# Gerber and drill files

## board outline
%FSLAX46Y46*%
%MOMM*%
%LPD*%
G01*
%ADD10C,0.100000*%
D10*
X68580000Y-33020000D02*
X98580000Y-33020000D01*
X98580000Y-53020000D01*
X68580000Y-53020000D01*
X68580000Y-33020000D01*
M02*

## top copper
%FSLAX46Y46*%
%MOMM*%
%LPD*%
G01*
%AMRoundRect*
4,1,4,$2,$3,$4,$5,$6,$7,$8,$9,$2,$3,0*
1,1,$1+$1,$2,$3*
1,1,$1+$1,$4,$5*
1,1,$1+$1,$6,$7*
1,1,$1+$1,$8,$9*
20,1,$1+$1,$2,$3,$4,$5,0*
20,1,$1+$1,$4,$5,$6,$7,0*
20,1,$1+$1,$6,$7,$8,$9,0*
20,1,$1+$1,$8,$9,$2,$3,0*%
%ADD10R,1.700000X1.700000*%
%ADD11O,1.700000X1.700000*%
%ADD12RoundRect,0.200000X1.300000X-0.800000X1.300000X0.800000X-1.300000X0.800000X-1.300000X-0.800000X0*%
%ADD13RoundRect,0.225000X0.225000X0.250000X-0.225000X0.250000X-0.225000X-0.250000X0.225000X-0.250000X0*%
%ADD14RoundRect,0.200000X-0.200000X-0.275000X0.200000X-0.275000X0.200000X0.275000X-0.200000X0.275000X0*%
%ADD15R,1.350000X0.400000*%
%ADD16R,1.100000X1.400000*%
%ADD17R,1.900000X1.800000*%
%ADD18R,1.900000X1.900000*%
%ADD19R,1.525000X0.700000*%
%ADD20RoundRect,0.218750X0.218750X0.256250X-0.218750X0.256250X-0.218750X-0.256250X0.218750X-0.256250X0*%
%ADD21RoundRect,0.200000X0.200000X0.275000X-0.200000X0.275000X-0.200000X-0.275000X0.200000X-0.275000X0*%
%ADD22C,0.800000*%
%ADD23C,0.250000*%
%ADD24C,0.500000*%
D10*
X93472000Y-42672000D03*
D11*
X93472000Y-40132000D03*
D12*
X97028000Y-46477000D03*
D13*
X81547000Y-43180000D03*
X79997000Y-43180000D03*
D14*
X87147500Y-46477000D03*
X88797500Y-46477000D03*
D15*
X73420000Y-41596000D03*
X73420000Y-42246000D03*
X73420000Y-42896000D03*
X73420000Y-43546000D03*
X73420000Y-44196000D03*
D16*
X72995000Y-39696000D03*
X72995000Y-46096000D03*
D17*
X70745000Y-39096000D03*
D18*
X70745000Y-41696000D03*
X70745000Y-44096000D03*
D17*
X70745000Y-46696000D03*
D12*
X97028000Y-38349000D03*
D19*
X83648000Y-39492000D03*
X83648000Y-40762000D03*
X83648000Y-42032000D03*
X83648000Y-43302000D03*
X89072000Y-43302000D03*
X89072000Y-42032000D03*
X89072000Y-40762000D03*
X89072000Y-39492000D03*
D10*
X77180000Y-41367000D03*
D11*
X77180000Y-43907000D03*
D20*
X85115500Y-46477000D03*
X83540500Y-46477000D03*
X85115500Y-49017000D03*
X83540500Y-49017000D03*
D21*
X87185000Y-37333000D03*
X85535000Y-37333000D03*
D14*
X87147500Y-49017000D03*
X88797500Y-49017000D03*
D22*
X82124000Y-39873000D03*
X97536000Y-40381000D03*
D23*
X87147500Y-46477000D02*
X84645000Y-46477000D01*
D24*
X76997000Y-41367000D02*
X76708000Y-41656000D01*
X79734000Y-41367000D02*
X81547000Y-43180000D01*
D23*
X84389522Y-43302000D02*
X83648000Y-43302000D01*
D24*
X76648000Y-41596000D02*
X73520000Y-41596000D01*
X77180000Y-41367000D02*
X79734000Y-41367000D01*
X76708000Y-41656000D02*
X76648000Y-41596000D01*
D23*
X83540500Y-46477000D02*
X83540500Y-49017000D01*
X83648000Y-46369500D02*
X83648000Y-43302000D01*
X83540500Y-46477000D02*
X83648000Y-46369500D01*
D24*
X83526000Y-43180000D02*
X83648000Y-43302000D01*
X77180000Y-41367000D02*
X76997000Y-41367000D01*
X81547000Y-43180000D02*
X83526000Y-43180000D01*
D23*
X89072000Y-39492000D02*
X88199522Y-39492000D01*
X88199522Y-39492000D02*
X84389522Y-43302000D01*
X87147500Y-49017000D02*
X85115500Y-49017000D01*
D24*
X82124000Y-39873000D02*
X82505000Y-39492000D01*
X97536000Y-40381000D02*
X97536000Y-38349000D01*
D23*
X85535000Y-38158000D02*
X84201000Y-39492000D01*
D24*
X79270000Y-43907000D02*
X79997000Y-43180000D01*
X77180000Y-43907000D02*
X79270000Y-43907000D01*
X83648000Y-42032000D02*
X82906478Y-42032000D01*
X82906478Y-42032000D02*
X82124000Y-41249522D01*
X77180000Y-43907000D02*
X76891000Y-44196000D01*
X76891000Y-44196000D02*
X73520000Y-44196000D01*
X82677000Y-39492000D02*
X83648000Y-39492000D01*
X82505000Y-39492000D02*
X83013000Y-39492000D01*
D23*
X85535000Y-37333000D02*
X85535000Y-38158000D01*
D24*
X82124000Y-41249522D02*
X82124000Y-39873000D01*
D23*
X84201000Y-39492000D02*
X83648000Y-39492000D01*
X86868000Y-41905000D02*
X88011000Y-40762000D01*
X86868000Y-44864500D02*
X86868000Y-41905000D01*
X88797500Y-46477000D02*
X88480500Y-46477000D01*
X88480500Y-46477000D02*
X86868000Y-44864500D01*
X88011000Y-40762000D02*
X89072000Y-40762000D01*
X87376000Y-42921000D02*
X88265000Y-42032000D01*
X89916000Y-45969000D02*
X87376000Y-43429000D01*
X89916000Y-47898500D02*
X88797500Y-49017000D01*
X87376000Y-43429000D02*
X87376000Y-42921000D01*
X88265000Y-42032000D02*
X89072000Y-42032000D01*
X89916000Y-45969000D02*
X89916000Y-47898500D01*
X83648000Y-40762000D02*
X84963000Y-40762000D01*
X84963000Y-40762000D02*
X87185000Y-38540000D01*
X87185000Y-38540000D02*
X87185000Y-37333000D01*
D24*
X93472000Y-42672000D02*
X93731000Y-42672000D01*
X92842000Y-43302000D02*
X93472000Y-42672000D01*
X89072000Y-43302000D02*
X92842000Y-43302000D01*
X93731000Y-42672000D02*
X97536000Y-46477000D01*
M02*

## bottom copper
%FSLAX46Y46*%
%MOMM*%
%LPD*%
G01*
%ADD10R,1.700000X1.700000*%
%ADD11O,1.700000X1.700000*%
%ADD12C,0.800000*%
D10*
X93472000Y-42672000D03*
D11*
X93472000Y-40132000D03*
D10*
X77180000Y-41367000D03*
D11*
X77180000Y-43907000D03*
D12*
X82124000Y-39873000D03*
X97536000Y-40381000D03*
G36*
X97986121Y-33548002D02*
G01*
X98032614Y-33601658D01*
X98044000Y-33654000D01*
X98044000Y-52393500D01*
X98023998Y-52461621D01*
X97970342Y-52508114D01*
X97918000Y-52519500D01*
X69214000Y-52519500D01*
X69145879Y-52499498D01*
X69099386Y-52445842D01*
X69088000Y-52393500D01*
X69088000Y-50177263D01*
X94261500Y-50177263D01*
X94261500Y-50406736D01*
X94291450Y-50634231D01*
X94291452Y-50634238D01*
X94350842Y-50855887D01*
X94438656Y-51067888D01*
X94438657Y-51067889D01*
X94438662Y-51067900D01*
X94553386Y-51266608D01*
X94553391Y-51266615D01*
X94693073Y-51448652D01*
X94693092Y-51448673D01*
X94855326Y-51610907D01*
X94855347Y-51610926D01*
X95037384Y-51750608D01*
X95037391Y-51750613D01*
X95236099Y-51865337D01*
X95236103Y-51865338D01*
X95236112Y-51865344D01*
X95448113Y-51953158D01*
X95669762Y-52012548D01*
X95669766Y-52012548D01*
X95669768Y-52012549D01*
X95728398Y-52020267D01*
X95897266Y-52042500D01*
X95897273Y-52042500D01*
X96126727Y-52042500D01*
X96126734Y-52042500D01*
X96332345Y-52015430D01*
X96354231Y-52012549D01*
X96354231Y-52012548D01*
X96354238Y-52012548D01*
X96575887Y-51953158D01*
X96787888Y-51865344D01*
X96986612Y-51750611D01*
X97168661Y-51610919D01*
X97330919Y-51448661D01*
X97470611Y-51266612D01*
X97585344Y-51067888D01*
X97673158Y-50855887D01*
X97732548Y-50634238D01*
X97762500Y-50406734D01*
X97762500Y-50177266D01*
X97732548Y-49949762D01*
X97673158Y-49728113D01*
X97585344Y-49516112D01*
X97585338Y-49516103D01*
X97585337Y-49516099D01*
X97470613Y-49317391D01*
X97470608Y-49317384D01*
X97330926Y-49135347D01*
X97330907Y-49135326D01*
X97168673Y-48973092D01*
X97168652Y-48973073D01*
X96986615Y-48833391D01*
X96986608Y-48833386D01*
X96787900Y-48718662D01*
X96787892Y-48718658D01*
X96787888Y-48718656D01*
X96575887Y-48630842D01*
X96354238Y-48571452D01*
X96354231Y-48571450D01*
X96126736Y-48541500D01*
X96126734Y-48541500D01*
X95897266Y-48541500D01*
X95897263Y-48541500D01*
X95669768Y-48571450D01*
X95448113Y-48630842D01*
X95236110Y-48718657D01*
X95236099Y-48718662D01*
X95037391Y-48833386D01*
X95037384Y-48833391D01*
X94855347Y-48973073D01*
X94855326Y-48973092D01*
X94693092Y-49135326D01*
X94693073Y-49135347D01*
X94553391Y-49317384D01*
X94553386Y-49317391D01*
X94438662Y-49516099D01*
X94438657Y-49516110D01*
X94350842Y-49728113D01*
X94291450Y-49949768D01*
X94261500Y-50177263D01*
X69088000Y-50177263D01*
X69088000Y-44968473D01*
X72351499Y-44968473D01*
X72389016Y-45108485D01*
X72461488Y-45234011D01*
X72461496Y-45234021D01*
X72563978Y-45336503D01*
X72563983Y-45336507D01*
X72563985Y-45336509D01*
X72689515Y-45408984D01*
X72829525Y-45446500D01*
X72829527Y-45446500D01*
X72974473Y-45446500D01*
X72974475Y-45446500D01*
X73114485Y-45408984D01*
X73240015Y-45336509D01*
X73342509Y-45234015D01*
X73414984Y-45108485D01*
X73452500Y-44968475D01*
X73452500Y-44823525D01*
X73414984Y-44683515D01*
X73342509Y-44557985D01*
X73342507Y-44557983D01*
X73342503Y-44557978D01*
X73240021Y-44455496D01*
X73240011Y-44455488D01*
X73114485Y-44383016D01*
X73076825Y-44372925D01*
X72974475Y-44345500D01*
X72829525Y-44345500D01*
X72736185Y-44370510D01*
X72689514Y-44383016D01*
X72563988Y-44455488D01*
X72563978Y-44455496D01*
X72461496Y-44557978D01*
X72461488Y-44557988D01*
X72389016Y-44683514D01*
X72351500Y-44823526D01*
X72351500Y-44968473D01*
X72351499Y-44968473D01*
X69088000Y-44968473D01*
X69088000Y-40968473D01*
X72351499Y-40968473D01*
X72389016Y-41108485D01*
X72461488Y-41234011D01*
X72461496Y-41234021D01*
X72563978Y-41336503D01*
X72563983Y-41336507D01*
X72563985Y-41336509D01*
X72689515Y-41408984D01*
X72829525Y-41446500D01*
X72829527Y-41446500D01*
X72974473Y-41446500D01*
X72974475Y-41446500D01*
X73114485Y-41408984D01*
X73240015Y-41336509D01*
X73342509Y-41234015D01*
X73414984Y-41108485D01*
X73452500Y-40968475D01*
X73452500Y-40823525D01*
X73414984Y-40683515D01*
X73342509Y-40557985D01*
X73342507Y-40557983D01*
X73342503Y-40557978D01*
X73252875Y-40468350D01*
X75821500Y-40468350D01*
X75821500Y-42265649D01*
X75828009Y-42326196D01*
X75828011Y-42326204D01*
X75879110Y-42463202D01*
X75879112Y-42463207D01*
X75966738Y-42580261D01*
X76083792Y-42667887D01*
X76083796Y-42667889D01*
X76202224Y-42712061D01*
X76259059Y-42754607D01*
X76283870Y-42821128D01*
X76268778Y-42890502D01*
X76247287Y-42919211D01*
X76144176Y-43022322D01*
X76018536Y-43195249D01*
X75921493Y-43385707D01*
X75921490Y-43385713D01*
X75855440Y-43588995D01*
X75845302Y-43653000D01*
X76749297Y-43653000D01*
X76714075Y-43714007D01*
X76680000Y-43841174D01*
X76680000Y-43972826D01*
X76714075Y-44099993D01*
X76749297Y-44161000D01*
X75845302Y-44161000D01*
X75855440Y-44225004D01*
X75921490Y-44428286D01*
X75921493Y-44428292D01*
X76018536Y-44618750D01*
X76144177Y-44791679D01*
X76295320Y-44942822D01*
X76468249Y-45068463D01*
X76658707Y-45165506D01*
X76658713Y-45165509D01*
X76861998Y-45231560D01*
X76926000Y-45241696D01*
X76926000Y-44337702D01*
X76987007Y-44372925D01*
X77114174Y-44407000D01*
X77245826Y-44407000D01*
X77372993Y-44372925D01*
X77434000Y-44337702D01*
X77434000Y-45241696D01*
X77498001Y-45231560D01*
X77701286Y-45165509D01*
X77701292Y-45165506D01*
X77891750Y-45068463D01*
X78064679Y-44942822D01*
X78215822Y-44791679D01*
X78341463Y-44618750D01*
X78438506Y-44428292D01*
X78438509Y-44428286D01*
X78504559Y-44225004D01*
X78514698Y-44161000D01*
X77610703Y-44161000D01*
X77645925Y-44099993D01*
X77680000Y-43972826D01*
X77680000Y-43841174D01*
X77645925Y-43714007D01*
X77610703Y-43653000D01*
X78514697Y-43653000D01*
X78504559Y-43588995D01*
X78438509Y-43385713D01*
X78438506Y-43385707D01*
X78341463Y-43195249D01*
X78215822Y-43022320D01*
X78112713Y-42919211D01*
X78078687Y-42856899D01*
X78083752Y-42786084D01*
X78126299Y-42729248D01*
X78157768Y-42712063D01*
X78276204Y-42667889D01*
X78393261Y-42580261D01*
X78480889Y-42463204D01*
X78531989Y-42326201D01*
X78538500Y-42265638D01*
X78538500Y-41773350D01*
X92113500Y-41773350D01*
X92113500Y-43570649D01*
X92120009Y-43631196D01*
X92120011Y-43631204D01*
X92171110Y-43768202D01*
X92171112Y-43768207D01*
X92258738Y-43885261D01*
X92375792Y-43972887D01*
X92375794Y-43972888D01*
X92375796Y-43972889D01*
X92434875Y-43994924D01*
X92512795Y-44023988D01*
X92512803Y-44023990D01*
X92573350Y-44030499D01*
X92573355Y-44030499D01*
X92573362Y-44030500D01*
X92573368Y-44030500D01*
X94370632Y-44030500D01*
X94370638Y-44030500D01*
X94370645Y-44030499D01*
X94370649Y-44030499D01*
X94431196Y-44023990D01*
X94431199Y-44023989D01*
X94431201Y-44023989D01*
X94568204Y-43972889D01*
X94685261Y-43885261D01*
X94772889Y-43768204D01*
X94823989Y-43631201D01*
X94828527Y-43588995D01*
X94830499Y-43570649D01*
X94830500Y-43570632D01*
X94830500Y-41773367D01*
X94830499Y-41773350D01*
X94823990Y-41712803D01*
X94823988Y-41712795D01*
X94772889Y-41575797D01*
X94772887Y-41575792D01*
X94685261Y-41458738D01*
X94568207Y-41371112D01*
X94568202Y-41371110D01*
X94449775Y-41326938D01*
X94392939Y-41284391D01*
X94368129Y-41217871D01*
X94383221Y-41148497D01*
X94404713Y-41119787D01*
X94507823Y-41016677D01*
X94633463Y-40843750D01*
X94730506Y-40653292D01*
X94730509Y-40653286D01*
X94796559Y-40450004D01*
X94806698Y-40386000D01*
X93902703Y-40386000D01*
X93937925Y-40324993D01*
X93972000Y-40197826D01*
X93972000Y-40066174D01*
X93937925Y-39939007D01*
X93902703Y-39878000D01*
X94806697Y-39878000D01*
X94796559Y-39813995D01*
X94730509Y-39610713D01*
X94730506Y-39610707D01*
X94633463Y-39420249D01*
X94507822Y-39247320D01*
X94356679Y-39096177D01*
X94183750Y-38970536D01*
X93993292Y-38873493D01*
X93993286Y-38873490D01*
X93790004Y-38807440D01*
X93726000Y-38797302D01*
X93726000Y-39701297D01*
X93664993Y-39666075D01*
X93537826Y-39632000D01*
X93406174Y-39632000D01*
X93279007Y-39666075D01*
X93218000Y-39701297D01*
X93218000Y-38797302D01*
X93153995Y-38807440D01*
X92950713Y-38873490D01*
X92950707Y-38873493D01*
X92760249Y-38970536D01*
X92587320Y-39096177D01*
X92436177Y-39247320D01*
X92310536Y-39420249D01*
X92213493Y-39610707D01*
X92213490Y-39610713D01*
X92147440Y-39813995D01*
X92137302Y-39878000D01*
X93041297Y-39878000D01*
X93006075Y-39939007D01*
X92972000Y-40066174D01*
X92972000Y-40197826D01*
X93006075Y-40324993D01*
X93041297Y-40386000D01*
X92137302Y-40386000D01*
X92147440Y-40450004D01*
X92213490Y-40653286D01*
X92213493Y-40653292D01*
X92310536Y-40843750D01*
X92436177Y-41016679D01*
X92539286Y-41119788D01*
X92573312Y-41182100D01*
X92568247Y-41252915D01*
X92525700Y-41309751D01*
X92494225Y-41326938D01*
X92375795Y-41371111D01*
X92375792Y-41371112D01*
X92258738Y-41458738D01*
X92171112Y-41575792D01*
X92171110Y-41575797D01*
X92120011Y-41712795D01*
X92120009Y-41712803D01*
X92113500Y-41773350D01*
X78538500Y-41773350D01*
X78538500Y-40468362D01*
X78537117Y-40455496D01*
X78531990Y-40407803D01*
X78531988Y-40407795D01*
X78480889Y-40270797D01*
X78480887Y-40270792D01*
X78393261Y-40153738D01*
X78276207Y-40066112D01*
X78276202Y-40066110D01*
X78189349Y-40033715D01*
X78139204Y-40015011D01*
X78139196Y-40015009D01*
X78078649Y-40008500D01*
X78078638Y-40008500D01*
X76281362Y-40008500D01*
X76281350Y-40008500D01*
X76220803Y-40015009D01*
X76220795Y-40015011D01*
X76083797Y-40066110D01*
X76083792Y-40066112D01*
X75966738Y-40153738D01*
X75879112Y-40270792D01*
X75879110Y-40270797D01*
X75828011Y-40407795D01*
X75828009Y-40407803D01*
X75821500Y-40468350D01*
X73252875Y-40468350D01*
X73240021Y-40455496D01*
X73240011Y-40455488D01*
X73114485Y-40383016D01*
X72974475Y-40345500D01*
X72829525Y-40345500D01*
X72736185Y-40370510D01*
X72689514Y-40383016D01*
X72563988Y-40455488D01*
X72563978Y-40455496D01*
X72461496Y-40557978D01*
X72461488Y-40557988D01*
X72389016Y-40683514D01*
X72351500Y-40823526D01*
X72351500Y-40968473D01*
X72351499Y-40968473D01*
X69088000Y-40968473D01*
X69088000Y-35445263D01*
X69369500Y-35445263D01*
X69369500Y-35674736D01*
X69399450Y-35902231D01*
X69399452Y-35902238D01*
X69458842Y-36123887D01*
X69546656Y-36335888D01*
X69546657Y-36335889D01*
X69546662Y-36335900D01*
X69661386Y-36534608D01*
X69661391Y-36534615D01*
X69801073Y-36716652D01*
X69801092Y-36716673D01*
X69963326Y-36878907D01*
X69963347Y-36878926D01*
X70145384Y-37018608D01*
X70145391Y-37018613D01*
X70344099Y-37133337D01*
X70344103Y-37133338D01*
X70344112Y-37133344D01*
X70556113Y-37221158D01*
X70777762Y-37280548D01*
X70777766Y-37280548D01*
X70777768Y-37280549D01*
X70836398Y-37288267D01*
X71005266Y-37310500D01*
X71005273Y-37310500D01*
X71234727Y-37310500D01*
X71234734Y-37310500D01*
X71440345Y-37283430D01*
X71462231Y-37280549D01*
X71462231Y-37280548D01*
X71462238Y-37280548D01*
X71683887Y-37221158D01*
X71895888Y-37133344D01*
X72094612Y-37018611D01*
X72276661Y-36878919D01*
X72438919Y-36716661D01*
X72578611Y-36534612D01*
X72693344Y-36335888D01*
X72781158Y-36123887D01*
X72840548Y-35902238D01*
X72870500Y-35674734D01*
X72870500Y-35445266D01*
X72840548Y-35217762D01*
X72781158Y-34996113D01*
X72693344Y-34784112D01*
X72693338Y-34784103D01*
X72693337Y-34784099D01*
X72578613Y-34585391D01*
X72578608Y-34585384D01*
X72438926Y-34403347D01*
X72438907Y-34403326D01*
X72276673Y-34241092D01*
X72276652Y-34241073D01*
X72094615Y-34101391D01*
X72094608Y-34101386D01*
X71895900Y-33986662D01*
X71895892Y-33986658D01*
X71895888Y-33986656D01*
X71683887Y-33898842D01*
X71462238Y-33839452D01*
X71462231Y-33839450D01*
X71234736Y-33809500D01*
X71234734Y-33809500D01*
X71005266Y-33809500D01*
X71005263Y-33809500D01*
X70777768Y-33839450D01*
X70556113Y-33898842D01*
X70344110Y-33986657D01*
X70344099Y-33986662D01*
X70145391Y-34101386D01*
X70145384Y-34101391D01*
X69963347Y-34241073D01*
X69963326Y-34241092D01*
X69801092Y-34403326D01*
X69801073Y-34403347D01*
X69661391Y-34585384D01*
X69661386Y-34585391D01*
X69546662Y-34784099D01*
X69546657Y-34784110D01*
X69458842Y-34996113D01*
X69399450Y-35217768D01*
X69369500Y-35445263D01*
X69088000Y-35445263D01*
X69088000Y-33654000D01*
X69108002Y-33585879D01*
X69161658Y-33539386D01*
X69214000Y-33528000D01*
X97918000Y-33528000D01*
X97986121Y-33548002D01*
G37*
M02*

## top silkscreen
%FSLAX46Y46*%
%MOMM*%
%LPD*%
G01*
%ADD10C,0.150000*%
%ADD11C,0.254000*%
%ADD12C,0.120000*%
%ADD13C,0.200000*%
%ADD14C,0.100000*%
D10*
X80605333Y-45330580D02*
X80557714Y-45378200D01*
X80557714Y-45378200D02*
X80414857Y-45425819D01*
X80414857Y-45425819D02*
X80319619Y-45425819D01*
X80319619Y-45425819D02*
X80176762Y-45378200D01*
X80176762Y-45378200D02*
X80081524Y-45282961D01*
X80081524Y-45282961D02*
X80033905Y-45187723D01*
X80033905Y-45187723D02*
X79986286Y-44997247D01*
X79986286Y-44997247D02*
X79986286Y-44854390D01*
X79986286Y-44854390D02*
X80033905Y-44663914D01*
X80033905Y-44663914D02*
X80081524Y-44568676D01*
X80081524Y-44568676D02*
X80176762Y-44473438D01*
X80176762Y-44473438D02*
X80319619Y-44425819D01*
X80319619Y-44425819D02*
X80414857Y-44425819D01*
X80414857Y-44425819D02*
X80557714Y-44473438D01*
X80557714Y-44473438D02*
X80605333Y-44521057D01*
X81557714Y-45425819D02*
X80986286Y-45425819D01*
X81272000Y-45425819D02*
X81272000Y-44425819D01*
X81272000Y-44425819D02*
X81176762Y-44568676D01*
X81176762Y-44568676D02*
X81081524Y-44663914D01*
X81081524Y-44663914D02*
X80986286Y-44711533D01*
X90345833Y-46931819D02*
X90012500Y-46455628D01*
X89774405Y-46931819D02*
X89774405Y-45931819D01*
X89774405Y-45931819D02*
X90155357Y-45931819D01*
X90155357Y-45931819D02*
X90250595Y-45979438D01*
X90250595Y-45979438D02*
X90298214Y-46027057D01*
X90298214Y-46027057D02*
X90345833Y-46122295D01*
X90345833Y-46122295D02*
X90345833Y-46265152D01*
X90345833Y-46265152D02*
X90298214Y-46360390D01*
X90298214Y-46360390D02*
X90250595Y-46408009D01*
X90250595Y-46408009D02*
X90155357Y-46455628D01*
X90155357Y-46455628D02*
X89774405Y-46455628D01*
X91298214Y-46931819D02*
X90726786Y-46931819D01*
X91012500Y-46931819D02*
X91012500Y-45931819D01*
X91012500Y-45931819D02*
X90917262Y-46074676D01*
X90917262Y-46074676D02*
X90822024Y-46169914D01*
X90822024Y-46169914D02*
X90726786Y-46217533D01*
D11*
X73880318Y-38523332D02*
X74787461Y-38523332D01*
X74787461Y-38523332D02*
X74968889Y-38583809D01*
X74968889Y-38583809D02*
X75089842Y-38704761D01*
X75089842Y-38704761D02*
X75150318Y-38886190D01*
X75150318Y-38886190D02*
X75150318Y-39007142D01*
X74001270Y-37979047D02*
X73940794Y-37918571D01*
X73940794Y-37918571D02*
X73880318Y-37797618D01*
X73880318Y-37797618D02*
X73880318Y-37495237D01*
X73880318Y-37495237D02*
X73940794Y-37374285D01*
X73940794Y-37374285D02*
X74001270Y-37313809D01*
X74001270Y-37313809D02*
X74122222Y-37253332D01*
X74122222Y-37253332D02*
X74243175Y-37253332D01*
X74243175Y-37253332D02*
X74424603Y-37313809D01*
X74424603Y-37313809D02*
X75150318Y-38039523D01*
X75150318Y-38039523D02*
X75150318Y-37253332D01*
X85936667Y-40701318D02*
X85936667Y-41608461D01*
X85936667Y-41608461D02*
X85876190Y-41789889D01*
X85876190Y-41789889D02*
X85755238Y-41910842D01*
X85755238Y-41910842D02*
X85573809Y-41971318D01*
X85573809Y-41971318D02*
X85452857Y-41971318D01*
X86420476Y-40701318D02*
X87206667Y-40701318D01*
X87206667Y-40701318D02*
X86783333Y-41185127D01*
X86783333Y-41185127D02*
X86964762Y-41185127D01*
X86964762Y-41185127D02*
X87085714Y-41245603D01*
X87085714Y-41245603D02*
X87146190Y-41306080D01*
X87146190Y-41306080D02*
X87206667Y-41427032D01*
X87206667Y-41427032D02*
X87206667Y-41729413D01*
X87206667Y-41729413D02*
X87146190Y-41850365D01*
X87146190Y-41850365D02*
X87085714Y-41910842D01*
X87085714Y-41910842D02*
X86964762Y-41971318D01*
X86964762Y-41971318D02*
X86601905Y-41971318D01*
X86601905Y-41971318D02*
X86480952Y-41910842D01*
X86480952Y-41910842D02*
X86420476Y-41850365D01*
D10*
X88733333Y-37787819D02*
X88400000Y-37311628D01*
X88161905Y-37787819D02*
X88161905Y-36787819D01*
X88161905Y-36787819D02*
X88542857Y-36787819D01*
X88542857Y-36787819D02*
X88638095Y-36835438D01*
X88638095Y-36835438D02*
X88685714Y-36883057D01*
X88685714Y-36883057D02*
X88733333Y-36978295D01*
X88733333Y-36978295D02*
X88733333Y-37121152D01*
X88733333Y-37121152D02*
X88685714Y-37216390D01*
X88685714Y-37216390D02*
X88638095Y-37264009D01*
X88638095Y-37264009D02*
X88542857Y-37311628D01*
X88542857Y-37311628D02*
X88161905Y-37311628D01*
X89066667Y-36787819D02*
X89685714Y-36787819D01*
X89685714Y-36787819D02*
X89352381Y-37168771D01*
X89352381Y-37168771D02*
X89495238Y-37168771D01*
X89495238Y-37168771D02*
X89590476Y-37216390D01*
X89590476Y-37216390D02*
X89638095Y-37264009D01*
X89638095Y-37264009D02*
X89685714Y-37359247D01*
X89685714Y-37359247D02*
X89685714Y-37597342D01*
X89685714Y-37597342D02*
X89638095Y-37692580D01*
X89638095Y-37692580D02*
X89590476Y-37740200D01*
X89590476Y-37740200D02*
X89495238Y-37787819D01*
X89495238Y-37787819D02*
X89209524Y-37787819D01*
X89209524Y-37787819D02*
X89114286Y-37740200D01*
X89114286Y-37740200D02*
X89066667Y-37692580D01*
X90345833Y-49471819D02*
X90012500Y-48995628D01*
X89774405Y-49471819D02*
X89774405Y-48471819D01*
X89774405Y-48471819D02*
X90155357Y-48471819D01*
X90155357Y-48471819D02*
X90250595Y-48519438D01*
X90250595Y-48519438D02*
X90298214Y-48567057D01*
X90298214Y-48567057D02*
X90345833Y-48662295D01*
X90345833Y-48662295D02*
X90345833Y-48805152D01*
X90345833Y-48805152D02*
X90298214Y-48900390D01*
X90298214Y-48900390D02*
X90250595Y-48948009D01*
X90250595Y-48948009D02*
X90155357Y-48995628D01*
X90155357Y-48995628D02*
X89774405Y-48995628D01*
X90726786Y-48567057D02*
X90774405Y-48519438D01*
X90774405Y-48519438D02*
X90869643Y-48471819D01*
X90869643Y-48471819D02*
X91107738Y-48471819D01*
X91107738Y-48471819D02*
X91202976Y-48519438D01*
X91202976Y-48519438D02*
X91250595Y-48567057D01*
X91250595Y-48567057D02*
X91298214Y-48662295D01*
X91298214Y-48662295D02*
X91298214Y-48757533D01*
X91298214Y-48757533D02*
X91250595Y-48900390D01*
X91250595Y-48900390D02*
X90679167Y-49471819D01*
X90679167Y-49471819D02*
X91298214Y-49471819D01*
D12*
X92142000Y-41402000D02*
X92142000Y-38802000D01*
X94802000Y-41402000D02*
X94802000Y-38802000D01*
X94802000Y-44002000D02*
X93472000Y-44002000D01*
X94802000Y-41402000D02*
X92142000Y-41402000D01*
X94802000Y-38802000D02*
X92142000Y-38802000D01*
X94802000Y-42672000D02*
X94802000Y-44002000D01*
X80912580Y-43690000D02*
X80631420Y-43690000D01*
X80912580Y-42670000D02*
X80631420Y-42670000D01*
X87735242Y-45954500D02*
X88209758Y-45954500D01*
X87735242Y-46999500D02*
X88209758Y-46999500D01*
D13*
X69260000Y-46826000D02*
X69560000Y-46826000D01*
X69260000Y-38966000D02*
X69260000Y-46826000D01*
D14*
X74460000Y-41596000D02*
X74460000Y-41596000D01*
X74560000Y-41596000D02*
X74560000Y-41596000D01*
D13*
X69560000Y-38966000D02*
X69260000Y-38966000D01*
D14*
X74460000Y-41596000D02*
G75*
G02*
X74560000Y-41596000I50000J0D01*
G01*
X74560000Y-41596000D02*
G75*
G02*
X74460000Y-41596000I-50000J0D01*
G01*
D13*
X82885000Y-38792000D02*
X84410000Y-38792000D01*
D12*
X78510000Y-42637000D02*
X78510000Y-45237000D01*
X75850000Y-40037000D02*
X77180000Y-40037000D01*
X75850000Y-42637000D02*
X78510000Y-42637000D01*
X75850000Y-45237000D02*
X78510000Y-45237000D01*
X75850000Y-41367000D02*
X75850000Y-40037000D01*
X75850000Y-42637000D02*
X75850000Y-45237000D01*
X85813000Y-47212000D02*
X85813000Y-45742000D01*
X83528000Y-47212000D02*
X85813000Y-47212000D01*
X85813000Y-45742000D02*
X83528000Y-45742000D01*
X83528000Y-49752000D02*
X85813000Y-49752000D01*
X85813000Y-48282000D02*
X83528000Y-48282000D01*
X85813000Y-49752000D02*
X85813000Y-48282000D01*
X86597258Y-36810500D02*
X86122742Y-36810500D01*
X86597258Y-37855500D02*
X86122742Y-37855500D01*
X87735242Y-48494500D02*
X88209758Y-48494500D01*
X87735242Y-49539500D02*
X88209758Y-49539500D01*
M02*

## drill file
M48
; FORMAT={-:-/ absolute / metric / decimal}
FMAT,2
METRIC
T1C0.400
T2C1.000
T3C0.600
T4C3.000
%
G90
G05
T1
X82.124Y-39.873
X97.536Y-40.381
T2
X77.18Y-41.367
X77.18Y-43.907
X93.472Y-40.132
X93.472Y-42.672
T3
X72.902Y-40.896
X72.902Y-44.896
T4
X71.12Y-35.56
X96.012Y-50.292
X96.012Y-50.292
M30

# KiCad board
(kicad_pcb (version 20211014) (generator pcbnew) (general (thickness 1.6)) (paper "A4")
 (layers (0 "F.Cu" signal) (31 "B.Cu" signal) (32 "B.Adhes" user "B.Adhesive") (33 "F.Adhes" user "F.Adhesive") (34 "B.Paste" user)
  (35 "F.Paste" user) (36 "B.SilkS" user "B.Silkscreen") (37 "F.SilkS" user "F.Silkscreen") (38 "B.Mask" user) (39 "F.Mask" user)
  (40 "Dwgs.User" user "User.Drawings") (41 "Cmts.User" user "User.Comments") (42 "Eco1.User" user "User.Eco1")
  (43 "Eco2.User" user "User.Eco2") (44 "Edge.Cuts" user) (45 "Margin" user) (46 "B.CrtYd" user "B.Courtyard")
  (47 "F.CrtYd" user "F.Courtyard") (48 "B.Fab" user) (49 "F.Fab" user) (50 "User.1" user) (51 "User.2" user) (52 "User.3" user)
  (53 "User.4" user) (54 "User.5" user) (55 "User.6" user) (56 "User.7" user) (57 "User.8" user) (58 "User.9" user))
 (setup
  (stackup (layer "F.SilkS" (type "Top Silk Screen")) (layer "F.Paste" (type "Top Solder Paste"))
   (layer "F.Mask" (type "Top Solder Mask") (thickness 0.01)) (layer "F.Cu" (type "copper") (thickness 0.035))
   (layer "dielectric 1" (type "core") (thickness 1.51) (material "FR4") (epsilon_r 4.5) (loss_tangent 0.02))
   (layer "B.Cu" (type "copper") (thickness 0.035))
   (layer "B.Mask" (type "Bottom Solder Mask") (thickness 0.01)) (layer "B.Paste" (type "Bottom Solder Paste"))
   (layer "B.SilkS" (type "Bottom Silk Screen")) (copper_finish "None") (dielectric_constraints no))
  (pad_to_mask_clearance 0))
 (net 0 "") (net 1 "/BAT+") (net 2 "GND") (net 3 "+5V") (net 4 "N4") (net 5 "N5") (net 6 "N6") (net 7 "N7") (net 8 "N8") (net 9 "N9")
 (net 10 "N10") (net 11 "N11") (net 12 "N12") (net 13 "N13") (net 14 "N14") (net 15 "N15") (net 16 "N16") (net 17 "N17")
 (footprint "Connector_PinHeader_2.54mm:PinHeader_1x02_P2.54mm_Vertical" (layer "F.Cu") (at 93.472 42.672 180)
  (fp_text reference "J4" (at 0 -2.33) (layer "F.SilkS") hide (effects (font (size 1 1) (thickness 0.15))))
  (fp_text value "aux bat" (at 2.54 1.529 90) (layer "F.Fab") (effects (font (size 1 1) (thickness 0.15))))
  (fp_line (start 1.33 1.27) (end 1.33 3.87) (layer "F.SilkS") (width 0.12))
  (fp_line (start -1.33 1.27) (end -1.33 3.87) (layer "F.SilkS") (width 0.12))
  (fp_line (start -1.33 -1.33) (end 0 -1.33) (layer "F.SilkS") (width 0.12))
  (fp_line (start -1.33 1.27) (end 1.33 1.27) (layer "F.SilkS") (width 0.12))
  (fp_line (start -1.33 3.87) (end 1.33 3.87) (layer "F.SilkS") (width 0.12))
  (fp_line (start -1.33 0) (end -1.33 -1.33) (layer "F.SilkS") (width 0.12))
  (pad "1" thru_hole rect (at 0 0 180) (size 1.7 1.7) (drill 1) (layers *.Cu *.Mask) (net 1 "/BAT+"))
  (pad "2" thru_hole oval (at 0 2.54 180) (size 1.7 1.7) (drill 1) (layers *.Cu *.Mask) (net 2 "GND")))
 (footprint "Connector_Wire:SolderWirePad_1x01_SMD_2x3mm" (layer "F.Cu") (at 97.028 46.477 90)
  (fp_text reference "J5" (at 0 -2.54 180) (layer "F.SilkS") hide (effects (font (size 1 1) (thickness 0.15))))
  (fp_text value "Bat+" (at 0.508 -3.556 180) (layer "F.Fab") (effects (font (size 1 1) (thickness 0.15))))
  (pad "1" smd roundrect (at 0 0 90) (size 2 3) (layers "F.Cu" "F.Paste" "F.Mask") (roundrect_rratio 0.1) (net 1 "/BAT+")))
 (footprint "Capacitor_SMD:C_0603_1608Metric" (layer "F.Cu") (at 80.772 43.18 180)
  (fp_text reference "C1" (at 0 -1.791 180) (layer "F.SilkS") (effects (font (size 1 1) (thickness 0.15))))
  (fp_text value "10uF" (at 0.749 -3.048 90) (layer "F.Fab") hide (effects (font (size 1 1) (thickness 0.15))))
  (fp_line (start -0.14058 -0.51) (end 0.14058 -0.51) (layer "F.SilkS") (width 0.12))
  (fp_line (start -0.14058 0.51) (end 0.14058 0.51) (layer "F.SilkS") (width 0.12))
  (pad "1" smd roundrect (at -0.775 0 180) (size 0.9 0.95) (layers "F.Cu" "F.Paste" "F.Mask") (roundrect_rratio 0.25) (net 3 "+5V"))
  (pad "2" smd roundrect (at 0.775 0 180) (size 0.9 0.95) (layers "F.Cu" "F.Paste" "F.Mask") (roundrect_rratio 0.25) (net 2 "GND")))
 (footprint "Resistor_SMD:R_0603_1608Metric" (layer "F.Cu") (at 87.9725 46.477)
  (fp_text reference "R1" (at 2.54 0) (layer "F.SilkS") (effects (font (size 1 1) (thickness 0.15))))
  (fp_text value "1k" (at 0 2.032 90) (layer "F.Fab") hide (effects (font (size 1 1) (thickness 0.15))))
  (fp_line (start -0.237258 -0.5225) (end 0.237258 -0.5225) (layer "F.SilkS") (width 0.12))
  (fp_line (start -0.237258 0.5225) (end 0.237258 0.5225) (layer "F.SilkS") (width 0.12))
  (pad "1" smd roundrect (at -0.825 0) (size 0.8 0.95) (layers "F.Cu" "F.Paste" "F.Mask") (roundrect_rratio 0.25) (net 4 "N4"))
  (pad "2" smd roundrect (at 0.825 0) (size 0.8 0.95) (layers "F.Cu" "F.Paste" "F.Mask") (roundrect_rratio 0.25) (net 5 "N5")))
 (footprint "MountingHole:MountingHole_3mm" (layer "F.Cu") (at 96.012 50.292)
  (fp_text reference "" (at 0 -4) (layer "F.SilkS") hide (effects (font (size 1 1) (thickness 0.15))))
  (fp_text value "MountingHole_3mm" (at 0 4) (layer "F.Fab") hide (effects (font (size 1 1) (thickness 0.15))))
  (pad "" np_thru_hole circle (at 0 0) (size 3 3) (drill 3) (layers *.Cu *.Mask))
  (pad "" np_thru_hole circle (at 0 0) (size 3 3) (drill 3) (layers *.Cu *.Mask)))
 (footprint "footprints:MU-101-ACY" (layer "F.Cu") (at 71.12 42.896 -90)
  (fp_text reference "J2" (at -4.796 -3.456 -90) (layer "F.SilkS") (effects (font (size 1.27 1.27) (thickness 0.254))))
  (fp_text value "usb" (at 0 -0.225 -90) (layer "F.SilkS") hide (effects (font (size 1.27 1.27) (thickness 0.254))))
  (fp_line (start 3.93 1.86) (end 3.93 1.56) (layer "F.SilkS") (width 0.2))
  (fp_line (start -3.93 1.86) (end 3.93 1.86) (layer "F.SilkS") (width 0.2))
  (fp_line (start -1.3 -3.34) (end -1.3 -3.34) (layer "F.SilkS") (width 0.1))
  (fp_line (start -1.3 -3.44) (end -1.3 -3.44) (layer "F.SilkS") (width 0.1))
  (fp_line (start -3.93 1.56) (end -3.93 1.86) (layer "F.SilkS") (width 0.2))
  (fp_arc (start -1.3 -3.34) (mid -1.35 -3.39) (end -1.3 -3.44) (layer "F.SilkS") (width 0.1))
  (fp_arc (start -1.3 -3.44) (mid -1.25 -3.39) (end -1.3 -3.34) (layer "F.SilkS") (width 0.1))
  (pad "" np_thru_hole circle (at -2 -1.782) (size 0.6 0.6) (drill 0.6) (layers F&B.Cu *.Mask))
  (pad "" np_thru_hole circle (at 2 -1.782) (size 0.6 0.6) (drill 0.6) (layers F&B.Cu *.Mask))
  (pad "1" smd rect (at -1.3 -2.3 270) (size 0.4 1.35) (layers "F.Cu" "F.Paste" "F.Mask") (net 3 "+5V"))
  (pad "2" smd rect (at -0.65 -2.3 270) (size 0.4 1.35) (layers "F.Cu" "F.Paste" "F.Mask") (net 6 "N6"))
  (pad "3" smd rect (at 0 -2.3 270) (size 0.4 1.35) (layers "F.Cu" "F.Paste" "F.Mask") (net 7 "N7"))
  (pad "4" smd rect (at 0.65 -2.3 270) (size 0.4 1.35) (layers "F.Cu" "F.Paste" "F.Mask") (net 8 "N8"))
  (pad "5" smd rect (at 1.3 -2.3 270) (size 0.4 1.35) (layers "F.Cu" "F.Paste" "F.Mask") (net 2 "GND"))
  (pad "MP1" smd rect (at -3.2 -1.875) (size 1.1 1.4) (layers "F.Cu" "F.Paste" "F.Mask") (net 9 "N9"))
  (pad "MP2" smd rect (at 3.2 -1.875) (size 1.1 1.4) (layers "F.Cu" "F.Paste" "F.Mask") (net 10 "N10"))
  (pad "MP3" smd rect (at -3.8 0.375 270) (size 1.8 1.9) (layers "F.Cu" "F.Paste" "F.Mask") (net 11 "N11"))
  (pad "MP4" smd rect (at -1.2 0.375 270) (size 1.9 1.9) (layers "F.Cu" "F.Paste" "F.Mask") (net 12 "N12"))
  (pad "MP5" smd rect (at 1.2 0.375 270) (size 1.9 1.9) (layers "F.Cu" "F.Paste" "F.Mask") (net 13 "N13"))
  (pad "MP6" smd rect (at 3.8 0.375 270) (size 1.8 1.9) (layers "F.Cu" "F.Paste" "F.Mask") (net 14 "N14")))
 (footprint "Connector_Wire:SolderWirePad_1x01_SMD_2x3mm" (layer "F.Cu") (at 97.028 38.349 90)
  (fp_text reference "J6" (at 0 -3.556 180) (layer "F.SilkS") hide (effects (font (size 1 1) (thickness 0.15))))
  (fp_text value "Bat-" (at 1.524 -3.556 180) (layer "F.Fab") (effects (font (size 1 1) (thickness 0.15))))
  (pad "1" smd roundrect (at 0 0 90) (size 2 3) (layers "F.Cu" "F.Paste" "F.Mask") (roundrect_rratio 0.1) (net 2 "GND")))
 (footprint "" (layer "F.Cu") (at 71.12 35.56)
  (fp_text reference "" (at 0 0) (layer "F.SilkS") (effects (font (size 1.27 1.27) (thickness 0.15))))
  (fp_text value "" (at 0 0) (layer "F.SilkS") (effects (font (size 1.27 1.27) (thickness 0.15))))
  (pad "" np_thru_hole circle (at 0 0) (size 3 3) (drill 3) (layers *.Cu *.Mask)))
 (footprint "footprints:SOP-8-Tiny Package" (layer "F.Cu") (at 86.36 41.397)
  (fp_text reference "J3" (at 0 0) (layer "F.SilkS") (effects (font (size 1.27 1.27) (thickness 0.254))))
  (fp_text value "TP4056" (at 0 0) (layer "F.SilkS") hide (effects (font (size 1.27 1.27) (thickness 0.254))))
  (fp_line (start -3.475 -2.605) (end -1.95 -2.605) (layer "F.SilkS") (width 0.2))
  (pad "1" smd rect (at -2.712 -1.905 90) (size 0.7 1.525) (layers "F.Cu" "F.Paste" "F.Mask") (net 2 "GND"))
  (pad "2" smd rect (at -2.712 -0.635 90) (size 0.7 1.525) (layers "F.Cu" "F.Paste" "F.Mask") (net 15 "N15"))
  (pad "3" smd rect (at -2.712 0.635 90) (size 0.7 1.525) (layers "F.Cu" "F.Paste" "F.Mask") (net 2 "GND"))
  (pad "4" smd rect (at -2.712 1.905 90) (size 0.7 1.525) (layers "F.Cu" "F.Paste" "F.Mask") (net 3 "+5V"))
  (pad "5" smd rect (at 2.712 1.905 90) (size 0.7 1.525) (layers "F.Cu" "F.Paste" "F.Mask") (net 1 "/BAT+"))
  (pad "6" smd rect (at 2.712 0.635 90) (size 0.7 1.525) (layers "F.Cu" "F.Paste" "F.Mask") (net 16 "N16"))
  (pad "7" smd rect (at 2.712 -0.635 90) (size 0.7 1.525) (layers "F.Cu" "F.Paste" "F.Mask") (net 5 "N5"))
  (pad "8" smd rect (at 2.712 -1.905 90) (size 0.7 1.525) (layers "F.Cu" "F.Paste" "F.Mask") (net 3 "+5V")))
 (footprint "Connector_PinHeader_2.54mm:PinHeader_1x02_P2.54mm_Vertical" (layer "F.Cu") (at 77.18 41.367)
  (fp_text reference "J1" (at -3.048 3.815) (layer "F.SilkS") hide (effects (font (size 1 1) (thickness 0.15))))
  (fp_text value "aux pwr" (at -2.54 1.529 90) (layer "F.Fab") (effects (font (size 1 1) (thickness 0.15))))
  (fp_line (start 1.33 1.27) (end 1.33 3.87) (layer "F.SilkS") (width 0.12))
  (fp_line (start -1.33 -1.33) (end 0 -1.33) (layer "F.SilkS") (width 0.12))
  (fp_line (start -1.33 1.27) (end 1.33 1.27) (layer "F.SilkS") (width 0.12))
  (fp_line (start -1.33 3.87) (end 1.33 3.87) (layer "F.SilkS") (width 0.12))
  (fp_line (start -1.33 0) (end -1.33 -1.33) (layer "F.SilkS") (width 0.12))
  (fp_line (start -1.33 1.27) (end -1.33 3.87) (layer "F.SilkS") (width 0.12))
  (pad "1" thru_hole rect (at 0 0) (size 1.7 1.7) (drill 1) (layers *.Cu *.Mask) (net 3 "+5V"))
  (pad "2" thru_hole oval (at 0 2.54) (size 1.7 1.7) (drill 1) (layers *.Cu *.Mask) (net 2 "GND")))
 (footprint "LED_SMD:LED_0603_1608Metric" (layer "F.Cu") (at 84.328 46.477 180)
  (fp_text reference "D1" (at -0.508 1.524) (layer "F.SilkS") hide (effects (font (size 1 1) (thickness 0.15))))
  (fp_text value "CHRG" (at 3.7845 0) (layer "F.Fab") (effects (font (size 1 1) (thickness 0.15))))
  (fp_line (start -1.485 -0.735) (end -1.485 0.735) (layer "F.SilkS") (width 0.12))
  (fp_line (start 0.8 -0.735) (end -1.485 -0.735) (layer "F.SilkS") (width 0.12))
  (fp_line (start -1.485 0.735) (end 0.8 0.735) (layer "F.SilkS") (width 0.12))
  (pad "1" smd roundrect (at -0.7875 0 180) (size 0.875 0.95) (layers "F.Cu" "F.Paste" "F.Mask") (roundrect_rratio 0.25) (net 4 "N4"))
  (pad "2" smd roundrect (at 0.7875 0 180) (size 0.875 0.95) (layers "F.Cu" "F.Paste" "F.Mask") (roundrect_rratio 0.25) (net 3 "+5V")))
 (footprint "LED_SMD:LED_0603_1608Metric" (layer "F.Cu") (at 84.328 49.017 180)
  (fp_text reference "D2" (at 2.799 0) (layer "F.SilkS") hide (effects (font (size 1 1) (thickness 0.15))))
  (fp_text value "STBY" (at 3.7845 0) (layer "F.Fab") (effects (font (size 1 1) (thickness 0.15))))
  (fp_line (start 0.8 -0.735) (end -1.485 -0.735) (layer "F.SilkS") (width 0.12))
  (fp_line (start -1.485 0.735) (end 0.8 0.735) (layer "F.SilkS") (width 0.12))
  (fp_line (start -1.485 -0.735) (end -1.485 0.735) (layer "F.SilkS") (width 0.12))
  (pad "1" smd roundrect (at -0.7875 0 180) (size 0.875 0.95) (layers "F.Cu" "F.Paste" "F.Mask") (roundrect_rratio 0.25) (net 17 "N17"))
  (pad "2" smd roundrect (at 0.7875 0 180) (size 0.875 0.95) (layers "F.Cu" "F.Paste" "F.Mask") (roundrect_rratio 0.25) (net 3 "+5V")))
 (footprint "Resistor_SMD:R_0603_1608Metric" (layer "F.Cu") (at 86.36 37.333 180)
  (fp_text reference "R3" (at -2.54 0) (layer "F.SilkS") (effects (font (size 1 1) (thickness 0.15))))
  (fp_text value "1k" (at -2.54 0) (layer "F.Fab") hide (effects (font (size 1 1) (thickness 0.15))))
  (fp_line (start -0.237258 0.5225) (end 0.237258 0.5225) (layer "F.SilkS") (width 0.12))
  (fp_line (start -0.237258 -0.5225) (end 0.237258 -0.5225) (layer "F.SilkS") (width 0.12))
  (pad "1" smd roundrect (at -0.825 0 180) (size 0.8 0.95) (layers "F.Cu" "F.Paste" "F.Mask") (roundrect_rratio 0.25) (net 15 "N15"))
  (pad "2" smd roundrect (at 0.825 0 180) (size 0.8 0.95) (layers "F.Cu" "F.Paste" "F.Mask") (roundrect_rratio 0.25) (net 2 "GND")))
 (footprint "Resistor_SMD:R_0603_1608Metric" (layer "F.Cu") (at 87.9725 49.017)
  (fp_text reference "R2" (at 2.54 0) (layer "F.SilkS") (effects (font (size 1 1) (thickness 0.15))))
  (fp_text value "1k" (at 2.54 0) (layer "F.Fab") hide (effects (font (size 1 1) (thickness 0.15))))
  (fp_line (start -0.237258 -0.5225) (end 0.237258 -0.5225) (layer "F.SilkS") (width 0.12))
  (fp_line (start -0.237258 0.5225) (end 0.237258 0.5225) (layer "F.SilkS") (width 0.12))
  (pad "1" smd roundrect (at -0.825 0) (size 0.8 0.95) (layers "F.Cu" "F.Paste" "F.Mask") (roundrect_rratio 0.25) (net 17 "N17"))
  (pad "2" smd roundrect (at 0.825 0) (size 0.8 0.95) (layers "F.Cu" "F.Paste" "F.Mask") (roundrect_rratio 0.25) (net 16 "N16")))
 (gr_rect (start 98.58 33.02) (end 68.58 53.02) (layer "Edge.Cuts") (width 0.1) (fill none))
 (segment (start 87.1475 46.477) (end 84.645 46.477) (width 0.25) (layer "F.Cu") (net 4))
 (segment (start 76.997 41.367) (end 76.708 41.656) (width 0.5) (layer "F.Cu") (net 3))
 (segment (start 79.734 41.367) (end 81.547 43.18) (width 0.5) (layer "F.Cu") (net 3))
 (segment (start 84.389522 43.302) (end 83.648 43.302) (width 0.25) (layer "F.Cu") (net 3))
 (segment (start 76.648 41.596) (end 73.52 41.596) (width 0.5) (layer "F.Cu") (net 3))
 (segment (start 77.18 41.367) (end 79.734 41.367) (width 0.5) (layer "F.Cu") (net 3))
 (segment (start 76.708 41.656) (end 76.648 41.596) (width 0.5) (layer "F.Cu") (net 3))
 (segment (start 83.5405 46.477) (end 83.5405 49.017) (width 0.25) (layer "F.Cu") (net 3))
 (segment (start 83.648 46.3695) (end 83.648 43.302) (width 0.25) (layer "F.Cu") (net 3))
 (segment (start 83.5405 46.477) (end 83.648 46.3695) (width 0.25) (layer "F.Cu") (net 3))
 (segment (start 83.526 43.18) (end 83.648 43.302) (width 0.5) (layer "F.Cu") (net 3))
 (segment (start 77.18 41.367) (end 76.997 41.367) (width 0.5) (layer "F.Cu") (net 3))
 (segment (start 81.547 43.18) (end 83.526 43.18) (width 0.5) (layer "F.Cu") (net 3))
 (segment (start 89.072 39.492) (end 88.199522 39.492) (width 0.25) (layer "F.Cu") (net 3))
 (segment (start 88.199522 39.492) (end 84.389522 43.302) (width 0.25) (layer "F.Cu") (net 3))
 (segment (start 87.1475 49.017) (end 85.1155 49.017) (width 0.25) (layer "F.Cu") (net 17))
 (segment (start 82.124 39.873) (end 82.505 39.492) (width 0.5) (layer "F.Cu") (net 2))
 (segment (start 97.536 40.381) (end 97.536 38.349) (width 0.5) (layer "F.Cu") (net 2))
 (segment (start 85.535 38.158) (end 84.201 39.492) (width 0.25) (layer "F.Cu") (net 2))
 (segment (start 79.27 43.907) (end 79.997 43.18) (width 0.5) (layer "F.Cu") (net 2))
 (segment (start 77.18 43.907) (end 79.27 43.907) (width 0.5) (layer "F.Cu") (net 2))
 (segment (start 83.648 42.032) (end 82.906478 42.032) (width 0.5) (layer "F.Cu") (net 2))
 (segment (start 82.906478 42.032) (end 82.124 41.249522) (width 0.5) (layer "F.Cu") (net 2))
 (segment (start 77.18 43.907) (end 76.891 44.196) (width 0.5) (layer "F.Cu") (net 2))
 (segment (start 76.891 44.196) (end 73.52 44.196) (width 0.5) (layer "F.Cu") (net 2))
 (segment (start 82.677 39.492) (end 83.648 39.492) (width 0.5) (layer "F.Cu") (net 2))
 (segment (start 82.505 39.492) (end 83.013 39.492) (width 0.5) (layer "F.Cu") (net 2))
 (segment (start 85.535 37.333) (end 85.535 38.158) (width 0.25) (layer "F.Cu") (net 2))
 (segment (start 82.124 41.249522) (end 82.124 39.873) (width 0.5) (layer "F.Cu") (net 2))
 (segment (start 84.201 39.492) (end 83.648 39.492) (width 0.25) (layer "F.Cu") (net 2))
 (via (at 82.124 39.873) (size 0.8) (drill 0.4) (layers "F.Cu" "B.Cu") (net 2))
 (via (at 97.536 40.381) (size 0.8) (drill 0.4) (layers "F.Cu" "B.Cu") (free) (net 2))
 (segment (start 86.868 41.905) (end 88.011 40.762) (width 0.25) (layer "F.Cu") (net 5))
 (segment (start 86.868 44.8645) (end 86.868 41.905) (width 0.25) (layer "F.Cu") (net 5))
 (segment (start 88.7975 46.477) (end 88.4805 46.477) (width 0.25) (layer "F.Cu") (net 5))
 (segment (start 88.4805 46.477) (end 86.868 44.8645) (width 0.25) (layer "F.Cu") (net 5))
 (segment (start 88.011 40.762) (end 89.072 40.762) (width 0.25) (layer "F.Cu") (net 5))
 (segment (start 87.376 42.921) (end 88.265 42.032) (width 0.25) (layer "F.Cu") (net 16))
 (segment (start 89.916 45.969) (end 87.376 43.429) (width 0.25) (layer "F.Cu") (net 16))
 (segment (start 89.916 47.8985) (end 88.7975 49.017) (width 0.25) (layer "F.Cu") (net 16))
 (segment (start 87.376 43.429) (end 87.376 42.921) (width 0.25) (layer "F.Cu") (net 16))
 (segment (start 88.265 42.032) (end 89.072 42.032) (width 0.25) (layer "F.Cu") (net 16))
 (segment (start 89.916 45.969) (end 89.916 47.8985) (width 0.25) (layer "F.Cu") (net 16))
 (segment (start 83.648 40.762) (end 84.963 40.762) (width 0.25) (layer "F.Cu") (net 15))
 (segment (start 84.963 40.762) (end 87.185 38.54) (width 0.25) (layer "F.Cu") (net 15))
 (segment (start 87.185 38.54) (end 87.185 37.333) (width 0.25) (layer "F.Cu") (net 15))
 (segment (start 93.472 42.672) (end 93.731 42.672) (width 0.5) (layer "F.Cu") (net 1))
 (segment (start 92.842 43.302) (end 93.472 42.672) (width 0.5) (layer "F.Cu") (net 1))
 (segment (start 89.072 43.302) (end 92.842 43.302) (width 0.5) (layer "F.Cu") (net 1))
 (segment (start 93.731 42.672) (end 97.536 46.477) (width 0.5) (layer "F.Cu") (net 1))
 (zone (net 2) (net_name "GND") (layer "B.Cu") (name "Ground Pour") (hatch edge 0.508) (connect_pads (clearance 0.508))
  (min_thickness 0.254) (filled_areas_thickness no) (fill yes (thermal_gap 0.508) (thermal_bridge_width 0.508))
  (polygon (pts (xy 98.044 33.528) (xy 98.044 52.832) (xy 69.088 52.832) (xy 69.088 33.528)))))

